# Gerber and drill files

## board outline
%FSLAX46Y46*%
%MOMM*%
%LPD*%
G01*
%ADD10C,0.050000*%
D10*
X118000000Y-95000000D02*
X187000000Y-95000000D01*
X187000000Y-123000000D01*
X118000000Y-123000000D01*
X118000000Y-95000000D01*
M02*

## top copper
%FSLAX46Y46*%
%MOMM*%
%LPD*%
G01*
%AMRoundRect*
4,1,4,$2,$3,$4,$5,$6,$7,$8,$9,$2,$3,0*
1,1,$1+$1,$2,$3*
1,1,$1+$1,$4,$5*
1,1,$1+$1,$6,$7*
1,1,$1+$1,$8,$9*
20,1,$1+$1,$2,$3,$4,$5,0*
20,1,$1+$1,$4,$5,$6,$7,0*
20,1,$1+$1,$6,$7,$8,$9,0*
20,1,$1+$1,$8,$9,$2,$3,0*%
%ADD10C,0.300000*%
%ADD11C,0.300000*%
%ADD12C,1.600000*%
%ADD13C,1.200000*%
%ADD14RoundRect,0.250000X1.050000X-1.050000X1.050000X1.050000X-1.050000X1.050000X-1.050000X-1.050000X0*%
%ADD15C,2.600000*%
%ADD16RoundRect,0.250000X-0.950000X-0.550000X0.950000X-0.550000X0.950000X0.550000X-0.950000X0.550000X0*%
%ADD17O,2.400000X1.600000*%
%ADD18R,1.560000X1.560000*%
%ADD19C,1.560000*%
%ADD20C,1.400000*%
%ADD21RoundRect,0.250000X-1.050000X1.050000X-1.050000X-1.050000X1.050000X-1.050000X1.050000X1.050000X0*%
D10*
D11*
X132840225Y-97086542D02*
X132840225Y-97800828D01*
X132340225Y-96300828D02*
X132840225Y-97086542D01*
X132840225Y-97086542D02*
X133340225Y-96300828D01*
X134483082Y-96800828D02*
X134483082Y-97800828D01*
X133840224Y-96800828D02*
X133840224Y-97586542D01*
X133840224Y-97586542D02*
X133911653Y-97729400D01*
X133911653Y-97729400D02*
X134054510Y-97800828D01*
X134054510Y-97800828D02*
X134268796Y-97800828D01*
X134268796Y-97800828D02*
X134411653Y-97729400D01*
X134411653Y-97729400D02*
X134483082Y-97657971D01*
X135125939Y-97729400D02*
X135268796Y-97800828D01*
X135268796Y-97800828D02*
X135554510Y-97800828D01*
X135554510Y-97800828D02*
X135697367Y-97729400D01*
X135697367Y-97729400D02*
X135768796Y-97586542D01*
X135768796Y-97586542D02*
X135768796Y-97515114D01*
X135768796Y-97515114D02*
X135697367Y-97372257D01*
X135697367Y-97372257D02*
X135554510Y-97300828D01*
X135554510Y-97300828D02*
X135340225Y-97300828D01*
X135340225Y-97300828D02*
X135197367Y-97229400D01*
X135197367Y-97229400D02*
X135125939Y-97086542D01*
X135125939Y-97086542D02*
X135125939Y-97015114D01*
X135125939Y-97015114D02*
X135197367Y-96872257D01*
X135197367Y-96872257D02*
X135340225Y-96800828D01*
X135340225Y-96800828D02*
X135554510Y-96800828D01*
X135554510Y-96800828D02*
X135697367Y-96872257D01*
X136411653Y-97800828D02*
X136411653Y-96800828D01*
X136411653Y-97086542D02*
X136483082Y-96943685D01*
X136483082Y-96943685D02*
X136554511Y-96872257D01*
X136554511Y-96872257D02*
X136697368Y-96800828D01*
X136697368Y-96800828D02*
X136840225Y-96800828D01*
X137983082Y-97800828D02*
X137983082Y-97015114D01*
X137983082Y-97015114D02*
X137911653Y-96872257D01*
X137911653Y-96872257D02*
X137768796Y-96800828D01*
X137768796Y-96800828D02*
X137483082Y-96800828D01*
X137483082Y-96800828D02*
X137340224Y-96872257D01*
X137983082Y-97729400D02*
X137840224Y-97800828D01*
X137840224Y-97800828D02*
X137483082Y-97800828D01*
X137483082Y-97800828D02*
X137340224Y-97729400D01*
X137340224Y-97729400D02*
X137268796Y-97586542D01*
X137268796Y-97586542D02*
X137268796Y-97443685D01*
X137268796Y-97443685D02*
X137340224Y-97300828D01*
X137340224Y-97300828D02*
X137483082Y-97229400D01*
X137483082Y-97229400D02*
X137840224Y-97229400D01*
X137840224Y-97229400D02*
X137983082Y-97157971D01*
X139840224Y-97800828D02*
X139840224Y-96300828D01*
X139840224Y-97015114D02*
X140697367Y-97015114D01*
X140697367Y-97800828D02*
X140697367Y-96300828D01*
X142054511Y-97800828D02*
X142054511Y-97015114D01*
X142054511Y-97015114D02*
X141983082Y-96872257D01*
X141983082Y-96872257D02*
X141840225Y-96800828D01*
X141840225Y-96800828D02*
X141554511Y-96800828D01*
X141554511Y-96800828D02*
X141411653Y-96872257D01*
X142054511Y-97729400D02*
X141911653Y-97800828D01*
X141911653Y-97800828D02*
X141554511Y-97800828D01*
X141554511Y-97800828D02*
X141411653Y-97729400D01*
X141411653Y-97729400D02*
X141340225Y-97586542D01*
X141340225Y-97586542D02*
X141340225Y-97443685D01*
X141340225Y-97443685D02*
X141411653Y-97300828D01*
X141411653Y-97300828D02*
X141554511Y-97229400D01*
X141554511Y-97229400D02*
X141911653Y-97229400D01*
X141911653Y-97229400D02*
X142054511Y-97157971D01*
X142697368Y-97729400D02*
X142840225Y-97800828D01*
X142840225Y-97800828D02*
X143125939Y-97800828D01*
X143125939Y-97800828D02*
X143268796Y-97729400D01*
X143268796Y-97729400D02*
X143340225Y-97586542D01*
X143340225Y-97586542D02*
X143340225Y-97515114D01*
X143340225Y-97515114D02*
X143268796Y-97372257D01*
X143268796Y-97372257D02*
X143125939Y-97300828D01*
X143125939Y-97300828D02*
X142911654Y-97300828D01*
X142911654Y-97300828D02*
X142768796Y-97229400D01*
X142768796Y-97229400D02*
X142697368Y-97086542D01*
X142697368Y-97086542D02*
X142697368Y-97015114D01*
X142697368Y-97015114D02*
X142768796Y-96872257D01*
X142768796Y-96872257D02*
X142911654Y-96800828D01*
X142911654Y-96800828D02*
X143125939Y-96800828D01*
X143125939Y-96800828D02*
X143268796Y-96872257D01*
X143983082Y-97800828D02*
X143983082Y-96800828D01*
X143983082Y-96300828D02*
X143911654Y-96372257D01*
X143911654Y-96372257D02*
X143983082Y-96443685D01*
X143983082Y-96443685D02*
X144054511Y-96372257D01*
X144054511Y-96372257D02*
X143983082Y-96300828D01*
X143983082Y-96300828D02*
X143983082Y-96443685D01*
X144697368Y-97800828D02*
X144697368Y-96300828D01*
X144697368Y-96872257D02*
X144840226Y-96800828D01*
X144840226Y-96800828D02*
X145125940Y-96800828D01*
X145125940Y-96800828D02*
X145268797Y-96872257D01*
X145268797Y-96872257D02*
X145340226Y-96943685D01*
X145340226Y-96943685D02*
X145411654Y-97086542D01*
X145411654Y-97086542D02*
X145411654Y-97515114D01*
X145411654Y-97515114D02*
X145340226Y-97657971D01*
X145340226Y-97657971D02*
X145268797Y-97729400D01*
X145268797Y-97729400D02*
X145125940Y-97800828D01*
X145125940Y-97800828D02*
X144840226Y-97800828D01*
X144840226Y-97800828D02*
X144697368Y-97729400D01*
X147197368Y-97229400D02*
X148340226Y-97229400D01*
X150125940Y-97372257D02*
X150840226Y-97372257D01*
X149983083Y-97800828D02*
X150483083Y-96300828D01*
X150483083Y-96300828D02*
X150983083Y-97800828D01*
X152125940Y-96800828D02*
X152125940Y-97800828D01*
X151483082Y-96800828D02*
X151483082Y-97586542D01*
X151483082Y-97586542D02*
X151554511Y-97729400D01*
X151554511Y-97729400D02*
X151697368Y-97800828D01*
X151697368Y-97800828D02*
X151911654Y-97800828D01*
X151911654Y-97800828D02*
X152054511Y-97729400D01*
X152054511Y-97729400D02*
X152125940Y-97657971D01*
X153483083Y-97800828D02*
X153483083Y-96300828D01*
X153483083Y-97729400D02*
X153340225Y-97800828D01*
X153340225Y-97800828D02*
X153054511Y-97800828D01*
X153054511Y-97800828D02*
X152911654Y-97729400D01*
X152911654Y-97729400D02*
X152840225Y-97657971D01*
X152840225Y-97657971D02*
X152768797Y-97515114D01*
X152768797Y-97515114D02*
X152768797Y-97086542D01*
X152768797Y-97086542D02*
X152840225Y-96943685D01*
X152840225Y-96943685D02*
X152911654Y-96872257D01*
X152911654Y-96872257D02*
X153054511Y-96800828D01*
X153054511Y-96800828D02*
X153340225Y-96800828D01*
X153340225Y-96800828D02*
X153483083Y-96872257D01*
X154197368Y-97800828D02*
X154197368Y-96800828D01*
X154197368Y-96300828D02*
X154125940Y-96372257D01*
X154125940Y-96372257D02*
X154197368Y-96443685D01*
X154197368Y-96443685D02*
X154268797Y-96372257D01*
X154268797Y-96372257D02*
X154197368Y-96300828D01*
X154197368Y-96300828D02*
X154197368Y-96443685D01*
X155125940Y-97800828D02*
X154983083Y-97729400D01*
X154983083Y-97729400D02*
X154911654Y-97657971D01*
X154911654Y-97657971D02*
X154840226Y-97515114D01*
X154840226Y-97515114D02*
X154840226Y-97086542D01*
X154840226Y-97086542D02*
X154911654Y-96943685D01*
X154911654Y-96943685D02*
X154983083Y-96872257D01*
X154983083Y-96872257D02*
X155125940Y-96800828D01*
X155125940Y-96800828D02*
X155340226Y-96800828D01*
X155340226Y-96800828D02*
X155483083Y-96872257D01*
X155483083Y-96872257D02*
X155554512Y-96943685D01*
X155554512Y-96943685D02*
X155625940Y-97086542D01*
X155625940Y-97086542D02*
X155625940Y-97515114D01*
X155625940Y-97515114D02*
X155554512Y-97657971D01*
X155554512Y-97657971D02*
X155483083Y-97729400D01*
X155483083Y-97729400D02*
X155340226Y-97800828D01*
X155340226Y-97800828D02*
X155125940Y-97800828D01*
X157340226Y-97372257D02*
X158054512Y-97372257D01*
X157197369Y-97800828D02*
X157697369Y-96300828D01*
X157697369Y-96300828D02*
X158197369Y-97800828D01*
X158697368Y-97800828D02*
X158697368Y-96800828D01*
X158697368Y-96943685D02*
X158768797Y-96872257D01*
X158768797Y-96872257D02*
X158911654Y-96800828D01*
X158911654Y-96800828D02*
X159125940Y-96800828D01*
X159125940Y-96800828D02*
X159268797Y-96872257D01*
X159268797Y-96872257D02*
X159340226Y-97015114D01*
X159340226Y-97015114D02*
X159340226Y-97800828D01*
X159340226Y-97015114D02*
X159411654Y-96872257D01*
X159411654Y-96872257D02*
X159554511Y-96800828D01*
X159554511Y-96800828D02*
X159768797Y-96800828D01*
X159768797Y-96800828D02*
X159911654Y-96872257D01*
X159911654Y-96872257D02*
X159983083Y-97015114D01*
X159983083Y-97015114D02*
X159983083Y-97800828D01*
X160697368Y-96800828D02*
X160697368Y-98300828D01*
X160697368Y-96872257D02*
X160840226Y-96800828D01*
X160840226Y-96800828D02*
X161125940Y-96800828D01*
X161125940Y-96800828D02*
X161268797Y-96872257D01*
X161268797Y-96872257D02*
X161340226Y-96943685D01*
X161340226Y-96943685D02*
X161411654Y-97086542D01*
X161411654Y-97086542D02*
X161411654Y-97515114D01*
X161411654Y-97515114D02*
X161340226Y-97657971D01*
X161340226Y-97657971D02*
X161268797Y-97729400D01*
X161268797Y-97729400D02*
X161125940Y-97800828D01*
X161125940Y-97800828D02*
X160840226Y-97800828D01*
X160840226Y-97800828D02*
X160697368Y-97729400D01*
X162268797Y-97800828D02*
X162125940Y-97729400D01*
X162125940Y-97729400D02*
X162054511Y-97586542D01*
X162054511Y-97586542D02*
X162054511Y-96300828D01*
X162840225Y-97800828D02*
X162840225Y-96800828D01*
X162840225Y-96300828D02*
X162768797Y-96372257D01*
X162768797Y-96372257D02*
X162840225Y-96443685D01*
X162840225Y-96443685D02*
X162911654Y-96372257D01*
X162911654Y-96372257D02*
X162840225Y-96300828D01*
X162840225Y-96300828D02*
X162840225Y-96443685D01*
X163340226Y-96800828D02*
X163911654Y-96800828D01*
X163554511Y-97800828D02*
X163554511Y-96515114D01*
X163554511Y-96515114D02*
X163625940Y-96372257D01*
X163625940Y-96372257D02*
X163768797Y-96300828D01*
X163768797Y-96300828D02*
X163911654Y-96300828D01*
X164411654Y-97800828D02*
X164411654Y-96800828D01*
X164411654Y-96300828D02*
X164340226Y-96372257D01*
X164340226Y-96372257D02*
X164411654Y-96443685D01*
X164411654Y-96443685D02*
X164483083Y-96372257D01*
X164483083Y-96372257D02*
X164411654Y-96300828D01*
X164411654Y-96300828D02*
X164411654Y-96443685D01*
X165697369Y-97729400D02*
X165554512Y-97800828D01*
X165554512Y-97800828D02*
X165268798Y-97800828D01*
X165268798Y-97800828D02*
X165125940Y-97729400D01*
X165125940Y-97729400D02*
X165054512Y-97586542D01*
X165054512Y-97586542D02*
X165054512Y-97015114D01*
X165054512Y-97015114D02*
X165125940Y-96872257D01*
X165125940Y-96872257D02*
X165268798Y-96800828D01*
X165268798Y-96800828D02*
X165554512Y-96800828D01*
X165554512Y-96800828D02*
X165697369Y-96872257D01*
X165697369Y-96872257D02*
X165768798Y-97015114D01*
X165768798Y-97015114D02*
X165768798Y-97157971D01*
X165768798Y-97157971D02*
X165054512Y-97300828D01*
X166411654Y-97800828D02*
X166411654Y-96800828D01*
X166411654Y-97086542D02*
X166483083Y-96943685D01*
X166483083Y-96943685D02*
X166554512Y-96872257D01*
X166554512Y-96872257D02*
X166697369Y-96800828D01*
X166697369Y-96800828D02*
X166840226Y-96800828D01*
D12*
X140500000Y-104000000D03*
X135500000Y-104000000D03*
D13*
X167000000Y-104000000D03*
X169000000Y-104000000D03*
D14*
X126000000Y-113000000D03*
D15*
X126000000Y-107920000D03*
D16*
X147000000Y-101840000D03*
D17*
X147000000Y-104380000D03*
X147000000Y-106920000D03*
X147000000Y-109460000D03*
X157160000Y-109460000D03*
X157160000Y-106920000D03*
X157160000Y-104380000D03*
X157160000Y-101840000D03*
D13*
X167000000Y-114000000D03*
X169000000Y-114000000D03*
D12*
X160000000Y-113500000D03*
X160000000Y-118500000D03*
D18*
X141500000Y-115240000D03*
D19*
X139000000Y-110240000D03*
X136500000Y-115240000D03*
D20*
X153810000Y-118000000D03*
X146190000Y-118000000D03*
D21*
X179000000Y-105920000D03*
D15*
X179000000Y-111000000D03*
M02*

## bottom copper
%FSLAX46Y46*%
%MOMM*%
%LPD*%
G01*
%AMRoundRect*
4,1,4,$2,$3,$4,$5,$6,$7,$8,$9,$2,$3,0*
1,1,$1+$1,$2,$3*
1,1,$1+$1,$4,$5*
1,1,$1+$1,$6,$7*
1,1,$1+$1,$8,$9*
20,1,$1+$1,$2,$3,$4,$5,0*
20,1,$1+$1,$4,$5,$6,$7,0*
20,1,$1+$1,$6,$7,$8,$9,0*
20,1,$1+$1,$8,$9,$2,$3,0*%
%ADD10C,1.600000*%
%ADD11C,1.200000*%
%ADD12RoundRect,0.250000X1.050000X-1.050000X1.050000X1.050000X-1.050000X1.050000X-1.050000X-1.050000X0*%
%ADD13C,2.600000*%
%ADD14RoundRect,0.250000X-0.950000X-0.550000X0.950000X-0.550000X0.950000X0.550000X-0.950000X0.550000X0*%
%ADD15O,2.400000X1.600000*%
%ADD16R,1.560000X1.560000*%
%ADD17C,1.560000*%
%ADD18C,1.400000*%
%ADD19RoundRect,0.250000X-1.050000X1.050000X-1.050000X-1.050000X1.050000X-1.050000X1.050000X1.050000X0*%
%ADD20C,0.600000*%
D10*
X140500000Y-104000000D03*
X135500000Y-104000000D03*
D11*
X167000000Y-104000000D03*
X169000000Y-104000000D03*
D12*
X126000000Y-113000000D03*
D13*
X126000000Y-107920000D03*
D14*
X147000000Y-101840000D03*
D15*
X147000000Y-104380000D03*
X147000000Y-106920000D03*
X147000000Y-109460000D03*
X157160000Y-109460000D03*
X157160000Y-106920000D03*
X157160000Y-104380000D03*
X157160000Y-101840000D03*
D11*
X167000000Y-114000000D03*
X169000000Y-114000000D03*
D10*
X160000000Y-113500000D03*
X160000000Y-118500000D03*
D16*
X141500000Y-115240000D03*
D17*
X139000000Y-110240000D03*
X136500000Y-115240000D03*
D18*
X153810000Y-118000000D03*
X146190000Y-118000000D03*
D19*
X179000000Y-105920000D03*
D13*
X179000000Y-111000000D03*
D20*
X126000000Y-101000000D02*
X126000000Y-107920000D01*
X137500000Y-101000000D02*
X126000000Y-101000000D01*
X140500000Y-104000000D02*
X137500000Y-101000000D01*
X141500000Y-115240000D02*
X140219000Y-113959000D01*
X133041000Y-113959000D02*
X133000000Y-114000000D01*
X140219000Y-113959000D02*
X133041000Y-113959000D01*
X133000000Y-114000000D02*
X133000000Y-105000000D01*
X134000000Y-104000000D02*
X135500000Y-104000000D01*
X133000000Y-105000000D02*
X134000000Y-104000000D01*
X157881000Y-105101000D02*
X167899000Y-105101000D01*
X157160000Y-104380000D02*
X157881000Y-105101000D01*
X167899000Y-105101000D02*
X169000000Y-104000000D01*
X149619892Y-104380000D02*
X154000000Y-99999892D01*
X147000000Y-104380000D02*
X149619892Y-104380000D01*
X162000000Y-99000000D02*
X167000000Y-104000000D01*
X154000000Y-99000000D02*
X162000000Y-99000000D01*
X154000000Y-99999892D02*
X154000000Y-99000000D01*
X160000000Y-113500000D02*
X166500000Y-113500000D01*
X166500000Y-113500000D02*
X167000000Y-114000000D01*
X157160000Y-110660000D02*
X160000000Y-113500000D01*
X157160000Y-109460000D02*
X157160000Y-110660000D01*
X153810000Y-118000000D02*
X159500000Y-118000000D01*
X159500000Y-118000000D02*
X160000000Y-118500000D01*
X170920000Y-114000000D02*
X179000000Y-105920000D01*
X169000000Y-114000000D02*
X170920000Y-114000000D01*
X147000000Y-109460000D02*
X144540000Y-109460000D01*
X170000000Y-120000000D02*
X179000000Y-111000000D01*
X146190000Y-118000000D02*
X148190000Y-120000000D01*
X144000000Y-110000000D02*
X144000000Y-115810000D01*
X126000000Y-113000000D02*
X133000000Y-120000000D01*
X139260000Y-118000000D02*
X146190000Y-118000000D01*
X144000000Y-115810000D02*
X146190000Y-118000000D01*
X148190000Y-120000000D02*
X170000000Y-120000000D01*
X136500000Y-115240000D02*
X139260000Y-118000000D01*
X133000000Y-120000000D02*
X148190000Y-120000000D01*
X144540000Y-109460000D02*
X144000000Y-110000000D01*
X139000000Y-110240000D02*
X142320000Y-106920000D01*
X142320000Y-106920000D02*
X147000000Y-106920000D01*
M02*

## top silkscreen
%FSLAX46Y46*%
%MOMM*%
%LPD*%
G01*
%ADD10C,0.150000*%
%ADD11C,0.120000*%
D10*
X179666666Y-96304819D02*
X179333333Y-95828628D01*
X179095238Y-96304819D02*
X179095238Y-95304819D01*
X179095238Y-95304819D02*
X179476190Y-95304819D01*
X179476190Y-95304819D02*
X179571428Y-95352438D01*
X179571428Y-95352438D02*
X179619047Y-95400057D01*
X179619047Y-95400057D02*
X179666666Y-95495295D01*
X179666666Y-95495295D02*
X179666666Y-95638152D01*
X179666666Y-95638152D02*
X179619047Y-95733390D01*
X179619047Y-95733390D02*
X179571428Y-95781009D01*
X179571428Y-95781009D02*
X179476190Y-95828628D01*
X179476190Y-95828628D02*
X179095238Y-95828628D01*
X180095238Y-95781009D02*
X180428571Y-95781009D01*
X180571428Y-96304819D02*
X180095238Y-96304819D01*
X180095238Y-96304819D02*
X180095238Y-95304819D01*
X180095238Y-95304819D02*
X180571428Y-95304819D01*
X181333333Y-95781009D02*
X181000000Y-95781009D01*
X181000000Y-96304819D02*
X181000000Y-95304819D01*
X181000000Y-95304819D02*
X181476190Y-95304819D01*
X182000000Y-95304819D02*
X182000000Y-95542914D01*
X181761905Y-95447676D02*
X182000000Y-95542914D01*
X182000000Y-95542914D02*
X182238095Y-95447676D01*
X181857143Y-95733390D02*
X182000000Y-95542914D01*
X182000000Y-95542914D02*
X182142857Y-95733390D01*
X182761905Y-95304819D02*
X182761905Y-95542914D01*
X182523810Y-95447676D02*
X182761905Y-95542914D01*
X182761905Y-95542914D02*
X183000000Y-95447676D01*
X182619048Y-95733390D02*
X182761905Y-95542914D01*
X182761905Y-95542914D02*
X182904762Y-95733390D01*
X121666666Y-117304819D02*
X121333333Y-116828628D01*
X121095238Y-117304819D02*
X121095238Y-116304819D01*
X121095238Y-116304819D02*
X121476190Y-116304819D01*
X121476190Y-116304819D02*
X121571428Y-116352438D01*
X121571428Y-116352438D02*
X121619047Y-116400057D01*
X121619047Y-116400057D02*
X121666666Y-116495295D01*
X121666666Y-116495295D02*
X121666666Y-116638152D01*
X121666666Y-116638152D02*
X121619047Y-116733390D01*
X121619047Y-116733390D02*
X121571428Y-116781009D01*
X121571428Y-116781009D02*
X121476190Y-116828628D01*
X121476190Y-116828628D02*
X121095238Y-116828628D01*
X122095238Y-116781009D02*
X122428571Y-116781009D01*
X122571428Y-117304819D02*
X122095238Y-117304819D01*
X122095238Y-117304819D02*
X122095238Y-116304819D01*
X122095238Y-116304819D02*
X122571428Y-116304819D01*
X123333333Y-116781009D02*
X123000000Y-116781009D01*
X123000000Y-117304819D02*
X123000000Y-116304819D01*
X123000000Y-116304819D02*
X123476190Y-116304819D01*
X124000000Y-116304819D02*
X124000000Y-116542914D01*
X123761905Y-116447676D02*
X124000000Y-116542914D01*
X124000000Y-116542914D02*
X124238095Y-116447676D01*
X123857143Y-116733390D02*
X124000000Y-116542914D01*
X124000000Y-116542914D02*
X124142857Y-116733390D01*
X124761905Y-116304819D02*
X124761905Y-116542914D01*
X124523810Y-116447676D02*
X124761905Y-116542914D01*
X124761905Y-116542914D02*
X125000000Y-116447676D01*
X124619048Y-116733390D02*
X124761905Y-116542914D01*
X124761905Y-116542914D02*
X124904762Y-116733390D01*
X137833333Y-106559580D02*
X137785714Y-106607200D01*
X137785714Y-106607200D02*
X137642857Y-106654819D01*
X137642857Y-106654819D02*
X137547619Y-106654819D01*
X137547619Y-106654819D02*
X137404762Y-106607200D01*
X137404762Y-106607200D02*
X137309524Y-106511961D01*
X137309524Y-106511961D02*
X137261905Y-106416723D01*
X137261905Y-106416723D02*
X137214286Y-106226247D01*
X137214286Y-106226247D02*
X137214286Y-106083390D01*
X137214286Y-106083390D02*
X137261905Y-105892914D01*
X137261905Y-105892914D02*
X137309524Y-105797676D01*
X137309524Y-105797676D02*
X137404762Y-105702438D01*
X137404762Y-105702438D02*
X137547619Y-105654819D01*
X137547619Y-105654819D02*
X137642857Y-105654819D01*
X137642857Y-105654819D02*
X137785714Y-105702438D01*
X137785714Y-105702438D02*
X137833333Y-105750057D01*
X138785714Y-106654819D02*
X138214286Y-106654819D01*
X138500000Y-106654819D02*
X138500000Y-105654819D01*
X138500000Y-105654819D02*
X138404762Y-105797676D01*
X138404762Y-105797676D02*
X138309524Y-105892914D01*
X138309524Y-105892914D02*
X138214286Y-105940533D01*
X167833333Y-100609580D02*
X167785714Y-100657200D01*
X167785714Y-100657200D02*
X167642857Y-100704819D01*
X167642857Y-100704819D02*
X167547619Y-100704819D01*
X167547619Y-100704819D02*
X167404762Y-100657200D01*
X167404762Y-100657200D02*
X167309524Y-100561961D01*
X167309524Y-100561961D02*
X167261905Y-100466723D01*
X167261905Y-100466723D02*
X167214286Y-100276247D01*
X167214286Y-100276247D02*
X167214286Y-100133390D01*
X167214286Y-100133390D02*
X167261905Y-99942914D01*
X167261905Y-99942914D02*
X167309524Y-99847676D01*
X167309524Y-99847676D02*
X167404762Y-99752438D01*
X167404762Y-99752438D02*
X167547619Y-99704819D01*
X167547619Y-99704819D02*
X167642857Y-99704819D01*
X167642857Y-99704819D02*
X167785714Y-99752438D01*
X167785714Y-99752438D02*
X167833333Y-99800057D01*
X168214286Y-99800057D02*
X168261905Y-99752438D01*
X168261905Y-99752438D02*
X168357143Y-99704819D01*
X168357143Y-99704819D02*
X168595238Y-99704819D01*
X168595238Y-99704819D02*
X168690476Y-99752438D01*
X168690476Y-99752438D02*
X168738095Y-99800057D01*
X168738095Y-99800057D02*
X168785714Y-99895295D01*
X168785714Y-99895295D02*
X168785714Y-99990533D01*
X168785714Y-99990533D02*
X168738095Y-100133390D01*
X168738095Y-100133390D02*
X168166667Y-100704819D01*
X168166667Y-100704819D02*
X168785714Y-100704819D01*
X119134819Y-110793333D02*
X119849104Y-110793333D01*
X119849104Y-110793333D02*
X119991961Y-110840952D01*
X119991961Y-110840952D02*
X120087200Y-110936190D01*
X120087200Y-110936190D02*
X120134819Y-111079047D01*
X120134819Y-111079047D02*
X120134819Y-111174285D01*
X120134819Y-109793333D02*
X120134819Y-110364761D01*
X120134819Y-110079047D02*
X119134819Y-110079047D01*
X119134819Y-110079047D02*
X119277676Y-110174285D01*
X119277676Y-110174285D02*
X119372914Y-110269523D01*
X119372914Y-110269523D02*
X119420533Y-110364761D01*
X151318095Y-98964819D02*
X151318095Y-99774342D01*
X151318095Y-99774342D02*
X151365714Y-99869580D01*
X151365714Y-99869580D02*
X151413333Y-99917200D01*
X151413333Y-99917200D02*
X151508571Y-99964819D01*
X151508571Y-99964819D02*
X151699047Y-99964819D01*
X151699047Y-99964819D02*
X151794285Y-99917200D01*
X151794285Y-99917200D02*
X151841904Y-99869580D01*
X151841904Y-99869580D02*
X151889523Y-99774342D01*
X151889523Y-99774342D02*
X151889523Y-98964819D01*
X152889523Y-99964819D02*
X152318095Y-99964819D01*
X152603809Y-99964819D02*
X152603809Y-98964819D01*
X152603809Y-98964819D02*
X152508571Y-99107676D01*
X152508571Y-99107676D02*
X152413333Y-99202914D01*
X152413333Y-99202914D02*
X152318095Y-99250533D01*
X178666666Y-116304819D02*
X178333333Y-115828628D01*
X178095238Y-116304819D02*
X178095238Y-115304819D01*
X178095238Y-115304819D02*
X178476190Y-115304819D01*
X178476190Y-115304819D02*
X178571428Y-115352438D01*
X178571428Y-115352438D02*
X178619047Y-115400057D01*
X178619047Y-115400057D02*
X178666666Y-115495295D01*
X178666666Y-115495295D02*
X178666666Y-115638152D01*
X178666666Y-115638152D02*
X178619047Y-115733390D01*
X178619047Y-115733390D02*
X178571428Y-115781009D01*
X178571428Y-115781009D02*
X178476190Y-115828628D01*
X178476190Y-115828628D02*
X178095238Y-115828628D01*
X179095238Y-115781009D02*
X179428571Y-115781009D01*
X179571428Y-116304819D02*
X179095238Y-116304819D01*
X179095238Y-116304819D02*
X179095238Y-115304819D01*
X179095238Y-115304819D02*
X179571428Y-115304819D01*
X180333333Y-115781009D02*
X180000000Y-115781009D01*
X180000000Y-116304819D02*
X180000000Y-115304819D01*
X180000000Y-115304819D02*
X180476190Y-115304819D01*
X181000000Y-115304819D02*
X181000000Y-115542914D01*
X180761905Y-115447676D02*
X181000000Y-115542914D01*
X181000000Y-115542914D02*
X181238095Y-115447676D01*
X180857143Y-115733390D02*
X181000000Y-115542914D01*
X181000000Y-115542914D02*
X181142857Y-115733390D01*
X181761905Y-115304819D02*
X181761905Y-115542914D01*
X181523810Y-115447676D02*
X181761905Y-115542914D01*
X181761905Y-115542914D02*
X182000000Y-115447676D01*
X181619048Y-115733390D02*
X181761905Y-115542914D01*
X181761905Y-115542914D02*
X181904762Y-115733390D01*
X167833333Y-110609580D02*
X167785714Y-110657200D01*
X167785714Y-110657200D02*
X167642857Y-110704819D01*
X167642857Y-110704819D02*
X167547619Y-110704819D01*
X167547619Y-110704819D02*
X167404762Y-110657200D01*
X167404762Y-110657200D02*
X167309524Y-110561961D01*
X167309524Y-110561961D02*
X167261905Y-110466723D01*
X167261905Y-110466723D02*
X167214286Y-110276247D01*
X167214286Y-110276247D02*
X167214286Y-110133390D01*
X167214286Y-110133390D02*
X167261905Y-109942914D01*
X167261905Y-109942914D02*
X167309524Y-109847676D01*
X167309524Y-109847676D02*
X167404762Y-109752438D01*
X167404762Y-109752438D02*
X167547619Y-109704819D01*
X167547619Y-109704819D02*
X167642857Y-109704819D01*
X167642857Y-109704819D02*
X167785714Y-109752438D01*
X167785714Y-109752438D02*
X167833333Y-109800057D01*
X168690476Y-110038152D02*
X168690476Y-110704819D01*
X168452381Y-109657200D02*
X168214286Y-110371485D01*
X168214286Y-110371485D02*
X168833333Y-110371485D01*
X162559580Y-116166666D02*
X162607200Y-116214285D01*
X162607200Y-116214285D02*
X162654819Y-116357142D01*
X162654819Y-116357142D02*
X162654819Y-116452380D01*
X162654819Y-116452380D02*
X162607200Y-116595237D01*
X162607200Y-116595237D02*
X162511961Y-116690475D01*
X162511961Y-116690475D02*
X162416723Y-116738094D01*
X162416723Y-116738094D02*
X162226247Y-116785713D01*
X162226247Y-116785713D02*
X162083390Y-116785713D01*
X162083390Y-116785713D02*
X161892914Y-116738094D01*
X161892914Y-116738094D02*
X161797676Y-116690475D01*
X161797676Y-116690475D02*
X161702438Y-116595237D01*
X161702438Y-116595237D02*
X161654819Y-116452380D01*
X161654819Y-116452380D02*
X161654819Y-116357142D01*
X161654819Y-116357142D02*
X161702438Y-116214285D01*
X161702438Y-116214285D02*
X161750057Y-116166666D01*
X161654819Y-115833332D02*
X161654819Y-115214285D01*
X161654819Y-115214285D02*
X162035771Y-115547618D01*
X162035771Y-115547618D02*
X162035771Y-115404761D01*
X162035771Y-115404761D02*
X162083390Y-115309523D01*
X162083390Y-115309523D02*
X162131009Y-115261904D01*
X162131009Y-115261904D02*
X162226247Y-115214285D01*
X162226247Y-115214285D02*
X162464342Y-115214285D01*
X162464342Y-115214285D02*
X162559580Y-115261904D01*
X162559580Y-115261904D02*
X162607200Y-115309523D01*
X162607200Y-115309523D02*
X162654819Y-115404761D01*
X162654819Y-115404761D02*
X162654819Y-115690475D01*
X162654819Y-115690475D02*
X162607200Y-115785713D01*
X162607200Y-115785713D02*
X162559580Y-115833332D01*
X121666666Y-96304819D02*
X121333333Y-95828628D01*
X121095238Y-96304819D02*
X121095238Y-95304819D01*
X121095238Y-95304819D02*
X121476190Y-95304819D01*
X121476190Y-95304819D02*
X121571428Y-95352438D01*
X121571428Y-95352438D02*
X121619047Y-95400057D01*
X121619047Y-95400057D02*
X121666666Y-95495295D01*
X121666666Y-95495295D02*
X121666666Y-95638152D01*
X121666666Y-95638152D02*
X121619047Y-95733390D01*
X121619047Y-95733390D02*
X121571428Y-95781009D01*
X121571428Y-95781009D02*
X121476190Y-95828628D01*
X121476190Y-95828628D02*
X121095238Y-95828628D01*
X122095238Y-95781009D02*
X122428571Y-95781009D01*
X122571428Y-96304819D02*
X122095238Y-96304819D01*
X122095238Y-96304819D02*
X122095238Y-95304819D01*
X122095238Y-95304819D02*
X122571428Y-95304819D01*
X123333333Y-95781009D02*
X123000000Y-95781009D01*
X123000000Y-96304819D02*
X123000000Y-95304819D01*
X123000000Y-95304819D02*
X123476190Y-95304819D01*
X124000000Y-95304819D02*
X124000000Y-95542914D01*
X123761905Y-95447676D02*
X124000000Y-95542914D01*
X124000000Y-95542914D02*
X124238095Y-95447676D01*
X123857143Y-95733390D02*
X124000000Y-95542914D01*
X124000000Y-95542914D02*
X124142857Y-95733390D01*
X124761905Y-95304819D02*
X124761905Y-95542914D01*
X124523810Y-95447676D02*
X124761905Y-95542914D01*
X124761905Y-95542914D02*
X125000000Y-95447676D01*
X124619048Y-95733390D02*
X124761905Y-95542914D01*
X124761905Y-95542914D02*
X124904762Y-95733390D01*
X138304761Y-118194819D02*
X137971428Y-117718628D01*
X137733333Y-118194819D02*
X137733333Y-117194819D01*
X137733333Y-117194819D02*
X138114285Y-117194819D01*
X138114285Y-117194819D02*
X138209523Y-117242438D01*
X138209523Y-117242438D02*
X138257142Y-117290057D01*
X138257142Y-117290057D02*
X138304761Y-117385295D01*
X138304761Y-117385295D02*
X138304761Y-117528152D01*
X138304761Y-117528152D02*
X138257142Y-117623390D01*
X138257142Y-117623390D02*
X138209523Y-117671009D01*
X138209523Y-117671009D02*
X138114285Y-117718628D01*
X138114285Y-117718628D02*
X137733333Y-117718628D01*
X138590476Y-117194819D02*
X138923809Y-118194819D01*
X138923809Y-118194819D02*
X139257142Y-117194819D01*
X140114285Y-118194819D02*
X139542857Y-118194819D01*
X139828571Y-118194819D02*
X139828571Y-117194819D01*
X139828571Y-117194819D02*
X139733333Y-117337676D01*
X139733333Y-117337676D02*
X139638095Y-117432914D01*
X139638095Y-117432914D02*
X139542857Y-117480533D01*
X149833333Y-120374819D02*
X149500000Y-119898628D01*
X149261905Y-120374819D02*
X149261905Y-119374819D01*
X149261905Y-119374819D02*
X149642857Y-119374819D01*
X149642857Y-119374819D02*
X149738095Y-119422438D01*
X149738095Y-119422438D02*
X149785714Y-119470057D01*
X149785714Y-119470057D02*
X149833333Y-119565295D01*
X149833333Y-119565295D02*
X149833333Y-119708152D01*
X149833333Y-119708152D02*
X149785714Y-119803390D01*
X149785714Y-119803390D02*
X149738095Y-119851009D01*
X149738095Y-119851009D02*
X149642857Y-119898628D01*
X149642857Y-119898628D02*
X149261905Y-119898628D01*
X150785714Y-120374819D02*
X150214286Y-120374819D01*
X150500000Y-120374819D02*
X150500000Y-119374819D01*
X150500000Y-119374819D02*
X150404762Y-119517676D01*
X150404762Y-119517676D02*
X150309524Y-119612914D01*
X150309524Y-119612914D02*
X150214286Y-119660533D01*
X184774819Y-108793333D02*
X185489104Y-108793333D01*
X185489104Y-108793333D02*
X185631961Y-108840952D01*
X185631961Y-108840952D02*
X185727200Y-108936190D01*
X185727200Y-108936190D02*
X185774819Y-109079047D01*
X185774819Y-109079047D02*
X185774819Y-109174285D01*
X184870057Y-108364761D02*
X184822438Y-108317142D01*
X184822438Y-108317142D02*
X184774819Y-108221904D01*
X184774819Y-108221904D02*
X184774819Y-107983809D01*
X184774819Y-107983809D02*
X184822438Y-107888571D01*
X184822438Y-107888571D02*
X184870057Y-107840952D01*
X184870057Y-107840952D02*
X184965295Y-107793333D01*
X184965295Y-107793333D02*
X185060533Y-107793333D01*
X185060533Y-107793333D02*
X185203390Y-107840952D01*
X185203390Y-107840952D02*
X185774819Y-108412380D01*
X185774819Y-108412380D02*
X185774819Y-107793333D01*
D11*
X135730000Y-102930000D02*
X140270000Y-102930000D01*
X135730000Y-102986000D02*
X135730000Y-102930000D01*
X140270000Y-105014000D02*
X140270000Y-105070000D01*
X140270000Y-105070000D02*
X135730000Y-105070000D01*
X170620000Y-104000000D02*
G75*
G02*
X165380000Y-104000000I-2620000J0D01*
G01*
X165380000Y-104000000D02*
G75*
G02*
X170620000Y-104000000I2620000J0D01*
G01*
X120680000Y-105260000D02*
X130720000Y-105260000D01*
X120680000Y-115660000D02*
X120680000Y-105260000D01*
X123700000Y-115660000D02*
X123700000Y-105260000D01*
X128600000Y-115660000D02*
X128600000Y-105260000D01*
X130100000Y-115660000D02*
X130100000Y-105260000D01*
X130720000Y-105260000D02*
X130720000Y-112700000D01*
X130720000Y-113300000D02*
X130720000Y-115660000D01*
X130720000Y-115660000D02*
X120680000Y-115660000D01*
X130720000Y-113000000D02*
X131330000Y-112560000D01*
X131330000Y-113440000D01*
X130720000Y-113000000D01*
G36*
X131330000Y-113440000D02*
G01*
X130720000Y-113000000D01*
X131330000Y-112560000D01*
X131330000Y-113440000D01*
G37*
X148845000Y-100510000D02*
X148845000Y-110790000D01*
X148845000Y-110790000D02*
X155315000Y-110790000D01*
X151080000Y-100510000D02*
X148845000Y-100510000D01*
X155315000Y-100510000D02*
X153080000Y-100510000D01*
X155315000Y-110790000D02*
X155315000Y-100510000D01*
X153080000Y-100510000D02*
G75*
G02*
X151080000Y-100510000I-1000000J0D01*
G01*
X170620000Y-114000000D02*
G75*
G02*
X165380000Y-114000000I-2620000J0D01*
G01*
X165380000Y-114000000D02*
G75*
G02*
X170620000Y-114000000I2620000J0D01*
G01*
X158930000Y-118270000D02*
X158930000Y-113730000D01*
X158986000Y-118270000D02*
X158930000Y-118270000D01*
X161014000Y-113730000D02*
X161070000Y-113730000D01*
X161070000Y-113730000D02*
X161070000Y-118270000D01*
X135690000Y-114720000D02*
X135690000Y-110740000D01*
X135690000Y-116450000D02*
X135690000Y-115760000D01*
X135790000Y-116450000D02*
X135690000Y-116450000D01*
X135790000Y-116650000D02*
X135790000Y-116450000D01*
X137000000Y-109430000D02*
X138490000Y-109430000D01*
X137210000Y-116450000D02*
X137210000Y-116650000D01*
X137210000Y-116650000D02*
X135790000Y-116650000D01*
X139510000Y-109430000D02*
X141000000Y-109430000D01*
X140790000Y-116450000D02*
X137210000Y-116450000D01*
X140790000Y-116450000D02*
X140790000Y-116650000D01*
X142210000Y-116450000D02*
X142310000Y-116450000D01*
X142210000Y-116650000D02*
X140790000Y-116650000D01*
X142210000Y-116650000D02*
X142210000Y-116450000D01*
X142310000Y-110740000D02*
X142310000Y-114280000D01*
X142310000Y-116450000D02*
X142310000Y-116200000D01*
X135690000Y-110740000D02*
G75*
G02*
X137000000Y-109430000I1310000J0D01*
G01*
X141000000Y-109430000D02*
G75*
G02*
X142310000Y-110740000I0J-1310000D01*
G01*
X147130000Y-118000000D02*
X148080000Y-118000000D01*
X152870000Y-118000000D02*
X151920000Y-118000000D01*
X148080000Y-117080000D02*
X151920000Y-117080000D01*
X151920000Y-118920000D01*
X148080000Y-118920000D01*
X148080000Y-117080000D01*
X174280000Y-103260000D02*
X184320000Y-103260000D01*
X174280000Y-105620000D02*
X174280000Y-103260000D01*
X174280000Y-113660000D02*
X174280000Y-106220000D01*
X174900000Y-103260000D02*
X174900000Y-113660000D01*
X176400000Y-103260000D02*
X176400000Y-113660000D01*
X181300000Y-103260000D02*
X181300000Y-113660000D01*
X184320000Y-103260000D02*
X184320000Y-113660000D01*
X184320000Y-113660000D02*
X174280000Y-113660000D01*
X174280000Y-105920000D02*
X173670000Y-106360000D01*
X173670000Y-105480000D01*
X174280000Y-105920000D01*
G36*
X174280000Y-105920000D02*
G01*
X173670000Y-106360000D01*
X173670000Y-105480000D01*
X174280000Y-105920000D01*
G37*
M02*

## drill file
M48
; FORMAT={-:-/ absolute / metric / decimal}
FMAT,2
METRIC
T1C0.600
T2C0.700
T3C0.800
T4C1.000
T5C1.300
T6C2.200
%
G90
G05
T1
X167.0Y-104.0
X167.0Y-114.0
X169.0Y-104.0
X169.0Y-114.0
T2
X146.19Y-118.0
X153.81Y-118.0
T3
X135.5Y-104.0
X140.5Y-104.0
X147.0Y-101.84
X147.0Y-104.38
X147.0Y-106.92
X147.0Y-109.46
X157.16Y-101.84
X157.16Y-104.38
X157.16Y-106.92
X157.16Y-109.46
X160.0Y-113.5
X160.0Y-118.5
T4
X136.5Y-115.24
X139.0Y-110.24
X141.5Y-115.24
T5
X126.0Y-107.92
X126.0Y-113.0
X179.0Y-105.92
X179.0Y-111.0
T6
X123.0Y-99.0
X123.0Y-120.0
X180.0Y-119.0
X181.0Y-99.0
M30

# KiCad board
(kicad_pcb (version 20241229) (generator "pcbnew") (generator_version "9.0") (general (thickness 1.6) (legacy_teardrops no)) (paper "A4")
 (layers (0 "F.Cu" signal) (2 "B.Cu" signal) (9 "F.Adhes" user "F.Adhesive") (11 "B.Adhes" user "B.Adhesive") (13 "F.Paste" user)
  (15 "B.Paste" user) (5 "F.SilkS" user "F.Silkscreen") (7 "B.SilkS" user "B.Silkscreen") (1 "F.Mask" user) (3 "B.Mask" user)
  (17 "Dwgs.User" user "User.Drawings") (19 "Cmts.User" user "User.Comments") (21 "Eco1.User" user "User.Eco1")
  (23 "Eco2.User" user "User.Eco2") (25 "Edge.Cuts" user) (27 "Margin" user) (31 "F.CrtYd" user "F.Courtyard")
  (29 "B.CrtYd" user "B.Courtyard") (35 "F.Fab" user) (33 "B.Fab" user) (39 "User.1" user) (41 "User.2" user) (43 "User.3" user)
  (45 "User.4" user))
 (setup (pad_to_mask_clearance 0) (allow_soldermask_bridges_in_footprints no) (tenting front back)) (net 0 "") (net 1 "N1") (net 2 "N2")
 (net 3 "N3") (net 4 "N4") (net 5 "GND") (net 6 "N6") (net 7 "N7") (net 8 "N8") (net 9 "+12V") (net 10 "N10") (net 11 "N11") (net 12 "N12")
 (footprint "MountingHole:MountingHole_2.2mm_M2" (layer "F.Cu") (at 181 99)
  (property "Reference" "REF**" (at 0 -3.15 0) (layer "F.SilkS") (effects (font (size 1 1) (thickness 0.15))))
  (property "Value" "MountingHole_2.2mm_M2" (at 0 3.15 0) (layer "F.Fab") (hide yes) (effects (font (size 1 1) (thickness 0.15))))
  (pad "" np_thru_hole circle (at 0 0) (size 2.2 2.2) (drill 2.2) (layers "*.Cu" "*.Mask")))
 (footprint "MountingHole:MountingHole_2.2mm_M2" (layer "F.Cu") (at 123 120)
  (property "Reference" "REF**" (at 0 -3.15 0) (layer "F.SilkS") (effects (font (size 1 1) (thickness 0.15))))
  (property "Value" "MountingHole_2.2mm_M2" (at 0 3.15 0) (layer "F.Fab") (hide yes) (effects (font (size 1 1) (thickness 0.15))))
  (pad "" np_thru_hole circle (at 0 0) (size 2.2 2.2) (drill 2.2) (layers "*.Cu" "*.Mask")))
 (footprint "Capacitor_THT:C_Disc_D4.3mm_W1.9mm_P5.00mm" (layer "F.Cu") (at 140.5 104 180)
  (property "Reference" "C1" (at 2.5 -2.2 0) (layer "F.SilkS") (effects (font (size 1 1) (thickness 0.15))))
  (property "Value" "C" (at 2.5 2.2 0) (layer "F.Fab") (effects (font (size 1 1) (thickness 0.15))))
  (fp_line (start 4.77 1.07) (end 0.23 1.07) (stroke (width 0.12) (type solid)) (layer "F.SilkS"))
  (fp_line (start 4.77 1.014) (end 4.77 1.07) (stroke (width 0.12) (type solid)) (layer "F.SilkS"))
  (fp_line (start 0.23 -1.014) (end 0.23 -1.07) (stroke (width 0.12) (type solid)) (layer "F.SilkS"))
  (fp_line (start 0.23 -1.07) (end 4.77 -1.07) (stroke (width 0.12) (type solid)) (layer "F.SilkS"))
  (pad "1" thru_hole circle (at 0 0 180) (size 1.6 1.6) (drill 0.8) (layers "*.Cu" "*.Mask") (remove_unused_layers no) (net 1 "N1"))
  (pad "2" thru_hole circle (at 5 0 180) (size 1.6 1.6) (drill 0.8) (layers "*.Cu" "*.Mask") (remove_unused_layers no) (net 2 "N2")))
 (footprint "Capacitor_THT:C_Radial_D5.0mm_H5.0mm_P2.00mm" (layer "F.Cu") (at 167 104)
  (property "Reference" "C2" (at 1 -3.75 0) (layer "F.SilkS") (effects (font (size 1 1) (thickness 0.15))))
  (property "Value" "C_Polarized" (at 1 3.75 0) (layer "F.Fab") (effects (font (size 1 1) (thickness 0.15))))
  (fp_circle (center 1 0) (end 3.62 0) (stroke (width 0.12) (type solid)) (fill no) (layer "F.SilkS"))
  (pad "1" thru_hole circle (at 0 0) (size 1.2 1.2) (drill 0.6) (layers "*.Cu" "*.Mask") (remove_unused_layers no) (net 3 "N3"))
  (pad "2" thru_hole circle (at 2 0) (size 1.2 1.2) (drill 0.6) (layers "*.Cu" "*.Mask") (remove_unused_layers no) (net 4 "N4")))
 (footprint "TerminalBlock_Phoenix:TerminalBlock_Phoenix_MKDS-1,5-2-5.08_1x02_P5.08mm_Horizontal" (layer "F.Cu") (at 126 113 90)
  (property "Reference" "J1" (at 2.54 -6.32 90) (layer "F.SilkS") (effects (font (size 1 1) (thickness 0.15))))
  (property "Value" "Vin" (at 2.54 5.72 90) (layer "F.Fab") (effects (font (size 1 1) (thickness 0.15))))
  (fp_line (start 7.74 -5.32) (end 7.74 4.72) (stroke (width 0.12) (type solid)) (layer "F.SilkS"))
  (fp_line (start -2.66 -5.32) (end 7.74 -5.32) (stroke (width 0.12) (type solid)) (layer "F.SilkS"))
  (fp_line (start -2.66 -2.3) (end 7.74 -2.3) (stroke (width 0.12) (type solid)) (layer "F.SilkS"))
  (fp_line (start -2.66 2.6) (end 7.74 2.6) (stroke (width 0.12) (type solid)) (layer "F.SilkS"))
  (fp_line (start -2.66 4.1) (end 7.74 4.1) (stroke (width 0.12) (type solid)) (layer "F.SilkS"))
  (fp_line (start 7.74 4.72) (end 0.3 4.72) (stroke (width 0.12) (type solid)) (layer "F.SilkS"))
  (fp_line (start -0.3 4.72) (end -2.66 4.72) (stroke (width 0.12) (type solid)) (layer "F.SilkS"))
  (fp_line (start -2.66 4.72) (end -2.66 -5.32) (stroke (width 0.12) (type solid)) (layer "F.SilkS"))
  (fp_poly (pts (xy 0 4.72) (xy 0.44 5.33) (xy -0.44 5.33)) (stroke (width 0.12) (type solid)) (fill yes) (layer "F.SilkS"))
  (pad "1" thru_hole roundrect (at 0 0 90) (size 2.6 2.6) (drill 1.3) (layers "*.Cu" "*.Mask") (remove_unused_layers no)
   (roundrect_rratio 0.096154) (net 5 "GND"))
  (pad "2" thru_hole circle (at 5.08 0 90) (size 2.6 2.6) (drill 1.3) (layers "*.Cu" "*.Mask") (remove_unused_layers no) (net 1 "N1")))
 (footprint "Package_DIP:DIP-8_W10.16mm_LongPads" (layer "F.Cu") (at 147 101.84)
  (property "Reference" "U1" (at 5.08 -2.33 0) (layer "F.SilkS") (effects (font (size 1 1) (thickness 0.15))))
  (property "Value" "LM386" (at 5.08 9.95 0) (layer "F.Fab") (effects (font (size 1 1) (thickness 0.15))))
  (fp_line (start 1.845 -1.33) (end 1.845 8.95) (stroke (width 0.12) (type solid)) (layer "F.SilkS"))
  (fp_line (start 1.845 8.95) (end 8.315 8.95) (stroke (width 0.12) (type solid)) (layer "F.SilkS"))
  (fp_line (start 4.08 -1.33) (end 1.845 -1.33) (stroke (width 0.12) (type solid)) (layer "F.SilkS"))
  (fp_line (start 8.315 -1.33) (end 6.08 -1.33) (stroke (width 0.12) (type solid)) (layer "F.SilkS"))
  (fp_line (start 8.315 8.95) (end 8.315 -1.33) (stroke (width 0.12) (type solid)) (layer "F.SilkS"))
  (fp_arc (start 6.08 -1.33) (mid 5.08 -0.33) (end 4.08 -1.33) (stroke (width 0.12) (type solid)) (layer "F.SilkS"))
  (pad "1" thru_hole roundrect (at 0 0) (size 2.4 1.6) (drill 0.8) (layers "*.Cu" "*.Mask") (remove_unused_layers no)
   (roundrect_rratio 0.15625) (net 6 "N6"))
  (pad "2" thru_hole oval (at 0 2.54) (size 2.4 1.6) (drill 0.8) (layers "*.Cu" "*.Mask") (remove_unused_layers no) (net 3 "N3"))
  (pad "3" thru_hole oval (at 0 5.08) (size 2.4 1.6) (drill 0.8) (layers "*.Cu" "*.Mask") (remove_unused_layers no) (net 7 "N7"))
  (pad "4" thru_hole oval (at 0 7.62) (size 2.4 1.6) (drill 0.8) (layers "*.Cu" "*.Mask") (remove_unused_layers no) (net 5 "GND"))
  (pad "5" thru_hole oval (at 10.16 7.62) (size 2.4 1.6) (drill 0.8) (layers "*.Cu" "*.Mask") (remove_unused_layers no) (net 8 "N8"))
  (pad "6" thru_hole oval (at 10.16 5.08) (size 2.4 1.6) (drill 0.8) (layers "*.Cu" "*.Mask") (remove_unused_layers no) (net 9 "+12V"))
  (pad "7" thru_hole oval (at 10.16 2.54) (size 2.4 1.6) (drill 0.8) (layers "*.Cu" "*.Mask") (remove_unused_layers no) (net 4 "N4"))
  (pad "8" thru_hole oval (at 10.16 0) (size 2.4 1.6) (drill 0.8) (layers "*.Cu" "*.Mask") (remove_unused_layers no) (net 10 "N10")))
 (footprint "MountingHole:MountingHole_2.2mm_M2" (layer "F.Cu") (at 180 119)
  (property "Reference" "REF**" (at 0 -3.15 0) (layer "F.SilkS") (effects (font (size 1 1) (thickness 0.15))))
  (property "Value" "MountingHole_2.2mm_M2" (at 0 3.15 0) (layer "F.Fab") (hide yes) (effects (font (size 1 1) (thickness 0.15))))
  (pad "" np_thru_hole circle (at 0 0) (size 2.2 2.2) (drill 2.2) (layers "*.Cu" "*.Mask")))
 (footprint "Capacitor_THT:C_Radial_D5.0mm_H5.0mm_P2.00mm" (layer "F.Cu") (at 167 114)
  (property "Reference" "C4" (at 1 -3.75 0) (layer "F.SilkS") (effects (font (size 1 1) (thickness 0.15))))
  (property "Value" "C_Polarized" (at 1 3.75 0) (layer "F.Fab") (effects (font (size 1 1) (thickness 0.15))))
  (fp_circle (center 1 0) (end 3.62 0) (stroke (width 0.12) (type solid)) (fill no) (layer "F.SilkS"))
  (pad "1" thru_hole circle (at 0 0) (size 1.2 1.2) (drill 0.6) (layers "*.Cu" "*.Mask") (remove_unused_layers no) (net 8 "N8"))
  (pad "2" thru_hole circle (at 2 0) (size 1.2 1.2) (drill 0.6) (layers "*.Cu" "*.Mask") (remove_unused_layers no) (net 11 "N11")))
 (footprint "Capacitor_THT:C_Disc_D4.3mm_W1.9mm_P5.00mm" (layer "F.Cu") (at 160 113.5 -90)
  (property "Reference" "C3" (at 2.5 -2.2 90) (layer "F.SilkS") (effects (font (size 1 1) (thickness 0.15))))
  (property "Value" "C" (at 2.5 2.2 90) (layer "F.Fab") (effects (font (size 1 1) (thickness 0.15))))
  (fp_line (start 4.77 1.07) (end 0.23 1.07) (stroke (width 0.12) (type solid)) (layer "F.SilkS"))
  (fp_line (start 4.77 1.014) (end 4.77 1.07) (stroke (width 0.12) (type solid)) (layer "F.SilkS"))
  (fp_line (start 0.23 -1.014) (end 0.23 -1.07) (stroke (width 0.12) (type solid)) (layer "F.SilkS"))
  (fp_line (start 0.23 -1.07) (end 4.77 -1.07) (stroke (width 0.12) (type solid)) (layer "F.SilkS"))
  (pad "1" thru_hole circle (at 0 0 270) (size 1.6 1.6) (drill 0.8) (layers "*.Cu" "*.Mask") (remove_unused_layers no) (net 8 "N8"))
  (pad "2" thru_hole circle (at 5 0 270) (size 1.6 1.6) (drill 0.8) (layers "*.Cu" "*.Mask") (remove_unused_layers no) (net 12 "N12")))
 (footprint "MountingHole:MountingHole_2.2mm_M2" (layer "F.Cu") (at 123 99)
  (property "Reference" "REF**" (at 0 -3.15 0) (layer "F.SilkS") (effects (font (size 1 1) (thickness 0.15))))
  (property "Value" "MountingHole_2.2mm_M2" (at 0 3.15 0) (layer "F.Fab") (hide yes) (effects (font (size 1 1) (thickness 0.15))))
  (pad "" np_thru_hole circle (at 0 0) (size 2.2 2.2) (drill 2.2) (layers "*.Cu" "*.Mask")))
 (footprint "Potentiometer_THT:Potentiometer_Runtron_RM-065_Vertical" (layer "F.Cu") (at 141.5 115.24 180)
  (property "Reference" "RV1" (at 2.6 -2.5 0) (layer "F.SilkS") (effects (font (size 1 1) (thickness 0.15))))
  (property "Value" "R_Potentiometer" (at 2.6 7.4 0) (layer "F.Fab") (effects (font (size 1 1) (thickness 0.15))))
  (fp_line (start 5.81 0.52) (end 5.81 4.5) (stroke (width 0.12) (type solid)) (layer "F.SilkS"))
  (fp_line (start 5.81 -1.21) (end 5.81 -0.52) (stroke (width 0.12) (type solid)) (layer "F.SilkS"))
  (fp_line (start 5.71 -1.21) (end 5.81 -1.21) (stroke (width 0.12) (type solid)) (layer "F.SilkS"))
  (fp_line (start 5.71 -1.41) (end 5.71 -1.21) (stroke (width 0.12) (type solid)) (layer "F.SilkS"))
  (fp_line (start 4.5 5.81) (end 3.01 5.81) (stroke (width 0.12) (type solid)) (layer "F.SilkS"))
  (fp_line (start 4.29 -1.21) (end 4.29 -1.41) (stroke (width 0.12) (type solid)) (layer "F.SilkS"))
  (fp_line (start 4.29 -1.41) (end 5.71 -1.41) (stroke (width 0.12) (type solid)) (layer "F.SilkS"))
  (fp_line (start 1.99 5.81) (end 0.5 5.81) (stroke (width 0.12) (type solid)) (layer "F.SilkS"))
  (fp_line (start 0.71 -1.21) (end 4.29 -1.21) (stroke (width 0.12) (type solid)) (layer "F.SilkS"))
  (fp_line (start 0.71 -1.21) (end 0.71 -1.41) (stroke (width 0.12) (type solid)) (layer "F.SilkS"))
  (fp_line (start -0.71 -1.21) (end -0.81 -1.21) (stroke (width 0.12) (type solid)) (layer "F.SilkS"))
  (fp_line (start -0.71 -1.41) (end 0.71 -1.41) (stroke (width 0.12) (type solid)) (layer "F.SilkS"))
  (fp_line (start -0.71 -1.41) (end -0.71 -1.21) (stroke (width 0.12) (type solid)) (layer "F.SilkS"))
  (fp_line (start -0.81 4.5) (end -0.81 0.96) (stroke (width 0.12) (type solid)) (layer "F.SilkS"))
  (fp_line (start -0.81 -1.21) (end -0.81 -0.96) (stroke (width 0.12) (type solid)) (layer "F.SilkS"))
  (fp_arc (start 5.81 4.5) (mid 5.42631 5.42631) (end 4.5 5.81) (stroke (width 0.12) (type solid)) (layer "F.SilkS"))
  (fp_arc (start 0.5 5.81) (mid -0.42631 5.42631) (end -0.81 4.5) (stroke (width 0.12) (type solid)) (layer "F.SilkS"))
  (pad "1" thru_hole rect (at 0 0 180) (size 1.56 1.56) (drill 1) (layers "*.Cu" "*.Mask") (remove_unused_layers no) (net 2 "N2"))
  (pad "2" thru_hole circle (at 2.5 5 180) (size 1.56 1.56) (drill 1) (layers "*.Cu" "*.Mask") (remove_unused_layers no) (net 7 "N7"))
  (pad "3" thru_hole circle (at 5 0 180) (size 1.56 1.56) (drill 1) (layers "*.Cu" "*.Mask") (remove_unused_layers no) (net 5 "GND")))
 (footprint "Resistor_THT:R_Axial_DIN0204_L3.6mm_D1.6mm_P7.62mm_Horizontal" (layer "F.Cu") (at 153.81 118 180)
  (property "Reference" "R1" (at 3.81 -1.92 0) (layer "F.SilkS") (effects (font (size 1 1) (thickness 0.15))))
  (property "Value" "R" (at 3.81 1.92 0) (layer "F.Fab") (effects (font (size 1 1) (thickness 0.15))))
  (fp_line (start 6.68 0) (end 5.73 0) (stroke (width 0.12) (type solid)) (layer "F.SilkS"))
  (fp_line (start 0.94 0) (end 1.89 0) (stroke (width 0.12) (type solid)) (layer "F.SilkS"))
  (fp_rect (start 1.89 -0.92) (end 5.73 0.92) (stroke (width 0.12) (type solid)) (fill no) (layer "F.SilkS"))
  (pad "1" thru_hole circle (at 0 0 180) (size 1.4 1.4) (drill 0.7) (layers "*.Cu" "*.Mask") (remove_unused_layers no) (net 12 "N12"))
  (pad "2" thru_hole circle (at 7.62 0 180) (size 1.4 1.4) (drill 0.7) (layers "*.Cu" "*.Mask") (remove_unused_layers no) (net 5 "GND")))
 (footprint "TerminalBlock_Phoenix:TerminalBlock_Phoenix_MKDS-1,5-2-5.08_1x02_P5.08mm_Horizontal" (layer "F.Cu") (at 179 105.92 -90)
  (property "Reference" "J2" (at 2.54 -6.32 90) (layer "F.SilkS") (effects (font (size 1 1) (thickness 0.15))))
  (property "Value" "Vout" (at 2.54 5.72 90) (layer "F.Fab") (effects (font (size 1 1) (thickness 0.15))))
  (fp_line (start -2.66 4.72) (end -2.66 -5.32) (stroke (width 0.12) (type solid)) (layer "F.SilkS"))
  (fp_line (start -0.3 4.72) (end -2.66 4.72) (stroke (width 0.12) (type solid)) (layer "F.SilkS"))
  (fp_line (start 7.74 4.72) (end 0.3 4.72) (stroke (width 0.12) (type solid)) (layer "F.SilkS"))
  (fp_line (start -2.66 4.1) (end 7.74 4.1) (stroke (width 0.12) (type solid)) (layer "F.SilkS"))
  (fp_line (start -2.66 2.6) (end 7.74 2.6) (stroke (width 0.12) (type solid)) (layer "F.SilkS"))
  (fp_line (start -2.66 -2.3) (end 7.74 -2.3) (stroke (width 0.12) (type solid)) (layer "F.SilkS"))
  (fp_line (start -2.66 -5.32) (end 7.74 -5.32) (stroke (width 0.12) (type solid)) (layer "F.SilkS"))
  (fp_line (start 7.74 -5.32) (end 7.74 4.72) (stroke (width 0.12) (type solid)) (layer "F.SilkS"))
  (fp_poly (pts (xy 0 4.72) (xy 0.44 5.33) (xy -0.44 5.33)) (stroke (width 0.12) (type solid)) (fill yes) (layer "F.SilkS"))
  (pad "1" thru_hole roundrect (at 0 0 270) (size 2.6 2.6) (drill 1.3) (layers "*.Cu" "*.Mask") (remove_unused_layers no)
   (roundrect_rratio 0.096154) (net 11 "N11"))
  (pad "2" thru_hole circle (at 5.08 0 270) (size 2.6 2.6) (drill 1.3) (layers "*.Cu" "*.Mask") (remove_unused_layers no) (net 5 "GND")))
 (gr_poly (pts (xy 118 95) (xy 187 95) (xy 187 123) (xy 118 123)) (stroke (width 0.05) (type solid)) (fill no) (layer "Edge.Cuts"))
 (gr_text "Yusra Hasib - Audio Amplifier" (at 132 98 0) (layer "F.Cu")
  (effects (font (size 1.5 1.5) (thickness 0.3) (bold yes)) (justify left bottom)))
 (segment (start 126 101) (end 126 107.92) (width 0.6) (layer "B.Cu") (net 1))
 (segment (start 137.5 101) (end 126 101) (width 0.6) (layer "B.Cu") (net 1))
 (segment (start 140.5 104) (end 137.5 101) (width 0.6) (layer "B.Cu") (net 1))
 (segment (start 141.5 115.24) (end 140.219 113.959) (width 0.6) (layer "B.Cu") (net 2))
 (segment (start 133.041 113.959) (end 133 114) (width 0.6) (layer "B.Cu") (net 2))
 (segment (start 140.219 113.959) (end 133.041 113.959) (width 0.6) (layer "B.Cu") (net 2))
 (segment (start 133 114) (end 133 105) (width 0.6) (layer "B.Cu") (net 2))
 (segment (start 134 104) (end 135.5 104) (width 0.6) (layer "B.Cu") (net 2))
 (segment (start 133 105) (end 134 104) (width 0.6) (layer "B.Cu") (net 2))
 (segment (start 157.881 105.101) (end 167.899 105.101) (width 0.6) (layer "B.Cu") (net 4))
 (segment (start 157.16 104.38) (end 157.881 105.101) (width 0.6) (layer "B.Cu") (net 4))
 (segment (start 167.899 105.101) (end 169 104) (width 0.6) (layer "B.Cu") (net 4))
 (segment (start 149.619892 104.38) (end 154 99.999892) (width 0.6) (layer "B.Cu") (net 3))
 (segment (start 147 104.38) (end 149.619892 104.38) (width 0.6) (layer "B.Cu") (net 3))
 (segment (start 162 99) (end 167 104) (width 0.6) (layer "B.Cu") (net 3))
 (segment (start 154 99) (end 162 99) (width 0.6) (layer "B.Cu") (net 3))
 (segment (start 154 99.999892) (end 154 99) (width 0.6) (layer "B.Cu") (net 3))
 (segment (start 160 113.5) (end 166.5 113.5) (width 0.6) (layer "B.Cu") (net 8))
 (segment (start 166.5 113.5) (end 167 114) (width 0.6) (layer "B.Cu") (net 8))
 (segment (start 157.16 110.66) (end 160 113.5) (width 0.6) (layer "B.Cu") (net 8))
 (segment (start 157.16 109.46) (end 157.16 110.66) (width 0.6) (layer "B.Cu") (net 8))
 (segment (start 153.81 118) (end 159.5 118) (width 0.6) (layer "B.Cu") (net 12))
 (segment (start 159.5 118) (end 160 118.5) (width 0.6) (layer "B.Cu") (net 12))
 (segment (start 170.92 114) (end 179 105.92) (width 0.6) (layer "B.Cu") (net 11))
 (segment (start 169 114) (end 170.92 114) (width 0.6) (layer "B.Cu") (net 11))
 (segment (start 147 109.46) (end 144.54 109.46) (width 0.6) (layer "B.Cu") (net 5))
 (segment (start 170 120) (end 179 111) (width 0.6) (layer "B.Cu") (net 5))
 (segment (start 146.19 118) (end 148.19 120) (width 0.6) (layer "B.Cu") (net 5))
 (segment (start 144 110) (end 144 115.81) (width 0.6) (layer "B.Cu") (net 5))
 (segment (start 126 113) (end 133 120) (width 0.6) (layer "B.Cu") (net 5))
 (segment (start 139.26 118) (end 146.19 118) (width 0.6) (layer "B.Cu") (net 5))
 (segment (start 144 115.81) (end 146.19 118) (width 0.6) (layer "B.Cu") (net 5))
 (segment (start 148.19 120) (end 170 120) (width 0.6) (layer "B.Cu") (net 5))
 (segment (start 136.5 115.24) (end 139.26 118) (width 0.6) (layer "B.Cu") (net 5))
 (segment (start 133 120) (end 148.19 120) (width 0.6) (layer "B.Cu") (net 5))
 (segment (start 144.54 109.46) (end 144 110) (width 0.6) (layer "B.Cu") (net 5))
 (segment (start 139 110.24) (end 142.32 106.92) (width 0.6) (layer "B.Cu") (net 7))
 (segment (start 142.32 106.92) (end 147 106.92) (width 0.6) (layer "B.Cu") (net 7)))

